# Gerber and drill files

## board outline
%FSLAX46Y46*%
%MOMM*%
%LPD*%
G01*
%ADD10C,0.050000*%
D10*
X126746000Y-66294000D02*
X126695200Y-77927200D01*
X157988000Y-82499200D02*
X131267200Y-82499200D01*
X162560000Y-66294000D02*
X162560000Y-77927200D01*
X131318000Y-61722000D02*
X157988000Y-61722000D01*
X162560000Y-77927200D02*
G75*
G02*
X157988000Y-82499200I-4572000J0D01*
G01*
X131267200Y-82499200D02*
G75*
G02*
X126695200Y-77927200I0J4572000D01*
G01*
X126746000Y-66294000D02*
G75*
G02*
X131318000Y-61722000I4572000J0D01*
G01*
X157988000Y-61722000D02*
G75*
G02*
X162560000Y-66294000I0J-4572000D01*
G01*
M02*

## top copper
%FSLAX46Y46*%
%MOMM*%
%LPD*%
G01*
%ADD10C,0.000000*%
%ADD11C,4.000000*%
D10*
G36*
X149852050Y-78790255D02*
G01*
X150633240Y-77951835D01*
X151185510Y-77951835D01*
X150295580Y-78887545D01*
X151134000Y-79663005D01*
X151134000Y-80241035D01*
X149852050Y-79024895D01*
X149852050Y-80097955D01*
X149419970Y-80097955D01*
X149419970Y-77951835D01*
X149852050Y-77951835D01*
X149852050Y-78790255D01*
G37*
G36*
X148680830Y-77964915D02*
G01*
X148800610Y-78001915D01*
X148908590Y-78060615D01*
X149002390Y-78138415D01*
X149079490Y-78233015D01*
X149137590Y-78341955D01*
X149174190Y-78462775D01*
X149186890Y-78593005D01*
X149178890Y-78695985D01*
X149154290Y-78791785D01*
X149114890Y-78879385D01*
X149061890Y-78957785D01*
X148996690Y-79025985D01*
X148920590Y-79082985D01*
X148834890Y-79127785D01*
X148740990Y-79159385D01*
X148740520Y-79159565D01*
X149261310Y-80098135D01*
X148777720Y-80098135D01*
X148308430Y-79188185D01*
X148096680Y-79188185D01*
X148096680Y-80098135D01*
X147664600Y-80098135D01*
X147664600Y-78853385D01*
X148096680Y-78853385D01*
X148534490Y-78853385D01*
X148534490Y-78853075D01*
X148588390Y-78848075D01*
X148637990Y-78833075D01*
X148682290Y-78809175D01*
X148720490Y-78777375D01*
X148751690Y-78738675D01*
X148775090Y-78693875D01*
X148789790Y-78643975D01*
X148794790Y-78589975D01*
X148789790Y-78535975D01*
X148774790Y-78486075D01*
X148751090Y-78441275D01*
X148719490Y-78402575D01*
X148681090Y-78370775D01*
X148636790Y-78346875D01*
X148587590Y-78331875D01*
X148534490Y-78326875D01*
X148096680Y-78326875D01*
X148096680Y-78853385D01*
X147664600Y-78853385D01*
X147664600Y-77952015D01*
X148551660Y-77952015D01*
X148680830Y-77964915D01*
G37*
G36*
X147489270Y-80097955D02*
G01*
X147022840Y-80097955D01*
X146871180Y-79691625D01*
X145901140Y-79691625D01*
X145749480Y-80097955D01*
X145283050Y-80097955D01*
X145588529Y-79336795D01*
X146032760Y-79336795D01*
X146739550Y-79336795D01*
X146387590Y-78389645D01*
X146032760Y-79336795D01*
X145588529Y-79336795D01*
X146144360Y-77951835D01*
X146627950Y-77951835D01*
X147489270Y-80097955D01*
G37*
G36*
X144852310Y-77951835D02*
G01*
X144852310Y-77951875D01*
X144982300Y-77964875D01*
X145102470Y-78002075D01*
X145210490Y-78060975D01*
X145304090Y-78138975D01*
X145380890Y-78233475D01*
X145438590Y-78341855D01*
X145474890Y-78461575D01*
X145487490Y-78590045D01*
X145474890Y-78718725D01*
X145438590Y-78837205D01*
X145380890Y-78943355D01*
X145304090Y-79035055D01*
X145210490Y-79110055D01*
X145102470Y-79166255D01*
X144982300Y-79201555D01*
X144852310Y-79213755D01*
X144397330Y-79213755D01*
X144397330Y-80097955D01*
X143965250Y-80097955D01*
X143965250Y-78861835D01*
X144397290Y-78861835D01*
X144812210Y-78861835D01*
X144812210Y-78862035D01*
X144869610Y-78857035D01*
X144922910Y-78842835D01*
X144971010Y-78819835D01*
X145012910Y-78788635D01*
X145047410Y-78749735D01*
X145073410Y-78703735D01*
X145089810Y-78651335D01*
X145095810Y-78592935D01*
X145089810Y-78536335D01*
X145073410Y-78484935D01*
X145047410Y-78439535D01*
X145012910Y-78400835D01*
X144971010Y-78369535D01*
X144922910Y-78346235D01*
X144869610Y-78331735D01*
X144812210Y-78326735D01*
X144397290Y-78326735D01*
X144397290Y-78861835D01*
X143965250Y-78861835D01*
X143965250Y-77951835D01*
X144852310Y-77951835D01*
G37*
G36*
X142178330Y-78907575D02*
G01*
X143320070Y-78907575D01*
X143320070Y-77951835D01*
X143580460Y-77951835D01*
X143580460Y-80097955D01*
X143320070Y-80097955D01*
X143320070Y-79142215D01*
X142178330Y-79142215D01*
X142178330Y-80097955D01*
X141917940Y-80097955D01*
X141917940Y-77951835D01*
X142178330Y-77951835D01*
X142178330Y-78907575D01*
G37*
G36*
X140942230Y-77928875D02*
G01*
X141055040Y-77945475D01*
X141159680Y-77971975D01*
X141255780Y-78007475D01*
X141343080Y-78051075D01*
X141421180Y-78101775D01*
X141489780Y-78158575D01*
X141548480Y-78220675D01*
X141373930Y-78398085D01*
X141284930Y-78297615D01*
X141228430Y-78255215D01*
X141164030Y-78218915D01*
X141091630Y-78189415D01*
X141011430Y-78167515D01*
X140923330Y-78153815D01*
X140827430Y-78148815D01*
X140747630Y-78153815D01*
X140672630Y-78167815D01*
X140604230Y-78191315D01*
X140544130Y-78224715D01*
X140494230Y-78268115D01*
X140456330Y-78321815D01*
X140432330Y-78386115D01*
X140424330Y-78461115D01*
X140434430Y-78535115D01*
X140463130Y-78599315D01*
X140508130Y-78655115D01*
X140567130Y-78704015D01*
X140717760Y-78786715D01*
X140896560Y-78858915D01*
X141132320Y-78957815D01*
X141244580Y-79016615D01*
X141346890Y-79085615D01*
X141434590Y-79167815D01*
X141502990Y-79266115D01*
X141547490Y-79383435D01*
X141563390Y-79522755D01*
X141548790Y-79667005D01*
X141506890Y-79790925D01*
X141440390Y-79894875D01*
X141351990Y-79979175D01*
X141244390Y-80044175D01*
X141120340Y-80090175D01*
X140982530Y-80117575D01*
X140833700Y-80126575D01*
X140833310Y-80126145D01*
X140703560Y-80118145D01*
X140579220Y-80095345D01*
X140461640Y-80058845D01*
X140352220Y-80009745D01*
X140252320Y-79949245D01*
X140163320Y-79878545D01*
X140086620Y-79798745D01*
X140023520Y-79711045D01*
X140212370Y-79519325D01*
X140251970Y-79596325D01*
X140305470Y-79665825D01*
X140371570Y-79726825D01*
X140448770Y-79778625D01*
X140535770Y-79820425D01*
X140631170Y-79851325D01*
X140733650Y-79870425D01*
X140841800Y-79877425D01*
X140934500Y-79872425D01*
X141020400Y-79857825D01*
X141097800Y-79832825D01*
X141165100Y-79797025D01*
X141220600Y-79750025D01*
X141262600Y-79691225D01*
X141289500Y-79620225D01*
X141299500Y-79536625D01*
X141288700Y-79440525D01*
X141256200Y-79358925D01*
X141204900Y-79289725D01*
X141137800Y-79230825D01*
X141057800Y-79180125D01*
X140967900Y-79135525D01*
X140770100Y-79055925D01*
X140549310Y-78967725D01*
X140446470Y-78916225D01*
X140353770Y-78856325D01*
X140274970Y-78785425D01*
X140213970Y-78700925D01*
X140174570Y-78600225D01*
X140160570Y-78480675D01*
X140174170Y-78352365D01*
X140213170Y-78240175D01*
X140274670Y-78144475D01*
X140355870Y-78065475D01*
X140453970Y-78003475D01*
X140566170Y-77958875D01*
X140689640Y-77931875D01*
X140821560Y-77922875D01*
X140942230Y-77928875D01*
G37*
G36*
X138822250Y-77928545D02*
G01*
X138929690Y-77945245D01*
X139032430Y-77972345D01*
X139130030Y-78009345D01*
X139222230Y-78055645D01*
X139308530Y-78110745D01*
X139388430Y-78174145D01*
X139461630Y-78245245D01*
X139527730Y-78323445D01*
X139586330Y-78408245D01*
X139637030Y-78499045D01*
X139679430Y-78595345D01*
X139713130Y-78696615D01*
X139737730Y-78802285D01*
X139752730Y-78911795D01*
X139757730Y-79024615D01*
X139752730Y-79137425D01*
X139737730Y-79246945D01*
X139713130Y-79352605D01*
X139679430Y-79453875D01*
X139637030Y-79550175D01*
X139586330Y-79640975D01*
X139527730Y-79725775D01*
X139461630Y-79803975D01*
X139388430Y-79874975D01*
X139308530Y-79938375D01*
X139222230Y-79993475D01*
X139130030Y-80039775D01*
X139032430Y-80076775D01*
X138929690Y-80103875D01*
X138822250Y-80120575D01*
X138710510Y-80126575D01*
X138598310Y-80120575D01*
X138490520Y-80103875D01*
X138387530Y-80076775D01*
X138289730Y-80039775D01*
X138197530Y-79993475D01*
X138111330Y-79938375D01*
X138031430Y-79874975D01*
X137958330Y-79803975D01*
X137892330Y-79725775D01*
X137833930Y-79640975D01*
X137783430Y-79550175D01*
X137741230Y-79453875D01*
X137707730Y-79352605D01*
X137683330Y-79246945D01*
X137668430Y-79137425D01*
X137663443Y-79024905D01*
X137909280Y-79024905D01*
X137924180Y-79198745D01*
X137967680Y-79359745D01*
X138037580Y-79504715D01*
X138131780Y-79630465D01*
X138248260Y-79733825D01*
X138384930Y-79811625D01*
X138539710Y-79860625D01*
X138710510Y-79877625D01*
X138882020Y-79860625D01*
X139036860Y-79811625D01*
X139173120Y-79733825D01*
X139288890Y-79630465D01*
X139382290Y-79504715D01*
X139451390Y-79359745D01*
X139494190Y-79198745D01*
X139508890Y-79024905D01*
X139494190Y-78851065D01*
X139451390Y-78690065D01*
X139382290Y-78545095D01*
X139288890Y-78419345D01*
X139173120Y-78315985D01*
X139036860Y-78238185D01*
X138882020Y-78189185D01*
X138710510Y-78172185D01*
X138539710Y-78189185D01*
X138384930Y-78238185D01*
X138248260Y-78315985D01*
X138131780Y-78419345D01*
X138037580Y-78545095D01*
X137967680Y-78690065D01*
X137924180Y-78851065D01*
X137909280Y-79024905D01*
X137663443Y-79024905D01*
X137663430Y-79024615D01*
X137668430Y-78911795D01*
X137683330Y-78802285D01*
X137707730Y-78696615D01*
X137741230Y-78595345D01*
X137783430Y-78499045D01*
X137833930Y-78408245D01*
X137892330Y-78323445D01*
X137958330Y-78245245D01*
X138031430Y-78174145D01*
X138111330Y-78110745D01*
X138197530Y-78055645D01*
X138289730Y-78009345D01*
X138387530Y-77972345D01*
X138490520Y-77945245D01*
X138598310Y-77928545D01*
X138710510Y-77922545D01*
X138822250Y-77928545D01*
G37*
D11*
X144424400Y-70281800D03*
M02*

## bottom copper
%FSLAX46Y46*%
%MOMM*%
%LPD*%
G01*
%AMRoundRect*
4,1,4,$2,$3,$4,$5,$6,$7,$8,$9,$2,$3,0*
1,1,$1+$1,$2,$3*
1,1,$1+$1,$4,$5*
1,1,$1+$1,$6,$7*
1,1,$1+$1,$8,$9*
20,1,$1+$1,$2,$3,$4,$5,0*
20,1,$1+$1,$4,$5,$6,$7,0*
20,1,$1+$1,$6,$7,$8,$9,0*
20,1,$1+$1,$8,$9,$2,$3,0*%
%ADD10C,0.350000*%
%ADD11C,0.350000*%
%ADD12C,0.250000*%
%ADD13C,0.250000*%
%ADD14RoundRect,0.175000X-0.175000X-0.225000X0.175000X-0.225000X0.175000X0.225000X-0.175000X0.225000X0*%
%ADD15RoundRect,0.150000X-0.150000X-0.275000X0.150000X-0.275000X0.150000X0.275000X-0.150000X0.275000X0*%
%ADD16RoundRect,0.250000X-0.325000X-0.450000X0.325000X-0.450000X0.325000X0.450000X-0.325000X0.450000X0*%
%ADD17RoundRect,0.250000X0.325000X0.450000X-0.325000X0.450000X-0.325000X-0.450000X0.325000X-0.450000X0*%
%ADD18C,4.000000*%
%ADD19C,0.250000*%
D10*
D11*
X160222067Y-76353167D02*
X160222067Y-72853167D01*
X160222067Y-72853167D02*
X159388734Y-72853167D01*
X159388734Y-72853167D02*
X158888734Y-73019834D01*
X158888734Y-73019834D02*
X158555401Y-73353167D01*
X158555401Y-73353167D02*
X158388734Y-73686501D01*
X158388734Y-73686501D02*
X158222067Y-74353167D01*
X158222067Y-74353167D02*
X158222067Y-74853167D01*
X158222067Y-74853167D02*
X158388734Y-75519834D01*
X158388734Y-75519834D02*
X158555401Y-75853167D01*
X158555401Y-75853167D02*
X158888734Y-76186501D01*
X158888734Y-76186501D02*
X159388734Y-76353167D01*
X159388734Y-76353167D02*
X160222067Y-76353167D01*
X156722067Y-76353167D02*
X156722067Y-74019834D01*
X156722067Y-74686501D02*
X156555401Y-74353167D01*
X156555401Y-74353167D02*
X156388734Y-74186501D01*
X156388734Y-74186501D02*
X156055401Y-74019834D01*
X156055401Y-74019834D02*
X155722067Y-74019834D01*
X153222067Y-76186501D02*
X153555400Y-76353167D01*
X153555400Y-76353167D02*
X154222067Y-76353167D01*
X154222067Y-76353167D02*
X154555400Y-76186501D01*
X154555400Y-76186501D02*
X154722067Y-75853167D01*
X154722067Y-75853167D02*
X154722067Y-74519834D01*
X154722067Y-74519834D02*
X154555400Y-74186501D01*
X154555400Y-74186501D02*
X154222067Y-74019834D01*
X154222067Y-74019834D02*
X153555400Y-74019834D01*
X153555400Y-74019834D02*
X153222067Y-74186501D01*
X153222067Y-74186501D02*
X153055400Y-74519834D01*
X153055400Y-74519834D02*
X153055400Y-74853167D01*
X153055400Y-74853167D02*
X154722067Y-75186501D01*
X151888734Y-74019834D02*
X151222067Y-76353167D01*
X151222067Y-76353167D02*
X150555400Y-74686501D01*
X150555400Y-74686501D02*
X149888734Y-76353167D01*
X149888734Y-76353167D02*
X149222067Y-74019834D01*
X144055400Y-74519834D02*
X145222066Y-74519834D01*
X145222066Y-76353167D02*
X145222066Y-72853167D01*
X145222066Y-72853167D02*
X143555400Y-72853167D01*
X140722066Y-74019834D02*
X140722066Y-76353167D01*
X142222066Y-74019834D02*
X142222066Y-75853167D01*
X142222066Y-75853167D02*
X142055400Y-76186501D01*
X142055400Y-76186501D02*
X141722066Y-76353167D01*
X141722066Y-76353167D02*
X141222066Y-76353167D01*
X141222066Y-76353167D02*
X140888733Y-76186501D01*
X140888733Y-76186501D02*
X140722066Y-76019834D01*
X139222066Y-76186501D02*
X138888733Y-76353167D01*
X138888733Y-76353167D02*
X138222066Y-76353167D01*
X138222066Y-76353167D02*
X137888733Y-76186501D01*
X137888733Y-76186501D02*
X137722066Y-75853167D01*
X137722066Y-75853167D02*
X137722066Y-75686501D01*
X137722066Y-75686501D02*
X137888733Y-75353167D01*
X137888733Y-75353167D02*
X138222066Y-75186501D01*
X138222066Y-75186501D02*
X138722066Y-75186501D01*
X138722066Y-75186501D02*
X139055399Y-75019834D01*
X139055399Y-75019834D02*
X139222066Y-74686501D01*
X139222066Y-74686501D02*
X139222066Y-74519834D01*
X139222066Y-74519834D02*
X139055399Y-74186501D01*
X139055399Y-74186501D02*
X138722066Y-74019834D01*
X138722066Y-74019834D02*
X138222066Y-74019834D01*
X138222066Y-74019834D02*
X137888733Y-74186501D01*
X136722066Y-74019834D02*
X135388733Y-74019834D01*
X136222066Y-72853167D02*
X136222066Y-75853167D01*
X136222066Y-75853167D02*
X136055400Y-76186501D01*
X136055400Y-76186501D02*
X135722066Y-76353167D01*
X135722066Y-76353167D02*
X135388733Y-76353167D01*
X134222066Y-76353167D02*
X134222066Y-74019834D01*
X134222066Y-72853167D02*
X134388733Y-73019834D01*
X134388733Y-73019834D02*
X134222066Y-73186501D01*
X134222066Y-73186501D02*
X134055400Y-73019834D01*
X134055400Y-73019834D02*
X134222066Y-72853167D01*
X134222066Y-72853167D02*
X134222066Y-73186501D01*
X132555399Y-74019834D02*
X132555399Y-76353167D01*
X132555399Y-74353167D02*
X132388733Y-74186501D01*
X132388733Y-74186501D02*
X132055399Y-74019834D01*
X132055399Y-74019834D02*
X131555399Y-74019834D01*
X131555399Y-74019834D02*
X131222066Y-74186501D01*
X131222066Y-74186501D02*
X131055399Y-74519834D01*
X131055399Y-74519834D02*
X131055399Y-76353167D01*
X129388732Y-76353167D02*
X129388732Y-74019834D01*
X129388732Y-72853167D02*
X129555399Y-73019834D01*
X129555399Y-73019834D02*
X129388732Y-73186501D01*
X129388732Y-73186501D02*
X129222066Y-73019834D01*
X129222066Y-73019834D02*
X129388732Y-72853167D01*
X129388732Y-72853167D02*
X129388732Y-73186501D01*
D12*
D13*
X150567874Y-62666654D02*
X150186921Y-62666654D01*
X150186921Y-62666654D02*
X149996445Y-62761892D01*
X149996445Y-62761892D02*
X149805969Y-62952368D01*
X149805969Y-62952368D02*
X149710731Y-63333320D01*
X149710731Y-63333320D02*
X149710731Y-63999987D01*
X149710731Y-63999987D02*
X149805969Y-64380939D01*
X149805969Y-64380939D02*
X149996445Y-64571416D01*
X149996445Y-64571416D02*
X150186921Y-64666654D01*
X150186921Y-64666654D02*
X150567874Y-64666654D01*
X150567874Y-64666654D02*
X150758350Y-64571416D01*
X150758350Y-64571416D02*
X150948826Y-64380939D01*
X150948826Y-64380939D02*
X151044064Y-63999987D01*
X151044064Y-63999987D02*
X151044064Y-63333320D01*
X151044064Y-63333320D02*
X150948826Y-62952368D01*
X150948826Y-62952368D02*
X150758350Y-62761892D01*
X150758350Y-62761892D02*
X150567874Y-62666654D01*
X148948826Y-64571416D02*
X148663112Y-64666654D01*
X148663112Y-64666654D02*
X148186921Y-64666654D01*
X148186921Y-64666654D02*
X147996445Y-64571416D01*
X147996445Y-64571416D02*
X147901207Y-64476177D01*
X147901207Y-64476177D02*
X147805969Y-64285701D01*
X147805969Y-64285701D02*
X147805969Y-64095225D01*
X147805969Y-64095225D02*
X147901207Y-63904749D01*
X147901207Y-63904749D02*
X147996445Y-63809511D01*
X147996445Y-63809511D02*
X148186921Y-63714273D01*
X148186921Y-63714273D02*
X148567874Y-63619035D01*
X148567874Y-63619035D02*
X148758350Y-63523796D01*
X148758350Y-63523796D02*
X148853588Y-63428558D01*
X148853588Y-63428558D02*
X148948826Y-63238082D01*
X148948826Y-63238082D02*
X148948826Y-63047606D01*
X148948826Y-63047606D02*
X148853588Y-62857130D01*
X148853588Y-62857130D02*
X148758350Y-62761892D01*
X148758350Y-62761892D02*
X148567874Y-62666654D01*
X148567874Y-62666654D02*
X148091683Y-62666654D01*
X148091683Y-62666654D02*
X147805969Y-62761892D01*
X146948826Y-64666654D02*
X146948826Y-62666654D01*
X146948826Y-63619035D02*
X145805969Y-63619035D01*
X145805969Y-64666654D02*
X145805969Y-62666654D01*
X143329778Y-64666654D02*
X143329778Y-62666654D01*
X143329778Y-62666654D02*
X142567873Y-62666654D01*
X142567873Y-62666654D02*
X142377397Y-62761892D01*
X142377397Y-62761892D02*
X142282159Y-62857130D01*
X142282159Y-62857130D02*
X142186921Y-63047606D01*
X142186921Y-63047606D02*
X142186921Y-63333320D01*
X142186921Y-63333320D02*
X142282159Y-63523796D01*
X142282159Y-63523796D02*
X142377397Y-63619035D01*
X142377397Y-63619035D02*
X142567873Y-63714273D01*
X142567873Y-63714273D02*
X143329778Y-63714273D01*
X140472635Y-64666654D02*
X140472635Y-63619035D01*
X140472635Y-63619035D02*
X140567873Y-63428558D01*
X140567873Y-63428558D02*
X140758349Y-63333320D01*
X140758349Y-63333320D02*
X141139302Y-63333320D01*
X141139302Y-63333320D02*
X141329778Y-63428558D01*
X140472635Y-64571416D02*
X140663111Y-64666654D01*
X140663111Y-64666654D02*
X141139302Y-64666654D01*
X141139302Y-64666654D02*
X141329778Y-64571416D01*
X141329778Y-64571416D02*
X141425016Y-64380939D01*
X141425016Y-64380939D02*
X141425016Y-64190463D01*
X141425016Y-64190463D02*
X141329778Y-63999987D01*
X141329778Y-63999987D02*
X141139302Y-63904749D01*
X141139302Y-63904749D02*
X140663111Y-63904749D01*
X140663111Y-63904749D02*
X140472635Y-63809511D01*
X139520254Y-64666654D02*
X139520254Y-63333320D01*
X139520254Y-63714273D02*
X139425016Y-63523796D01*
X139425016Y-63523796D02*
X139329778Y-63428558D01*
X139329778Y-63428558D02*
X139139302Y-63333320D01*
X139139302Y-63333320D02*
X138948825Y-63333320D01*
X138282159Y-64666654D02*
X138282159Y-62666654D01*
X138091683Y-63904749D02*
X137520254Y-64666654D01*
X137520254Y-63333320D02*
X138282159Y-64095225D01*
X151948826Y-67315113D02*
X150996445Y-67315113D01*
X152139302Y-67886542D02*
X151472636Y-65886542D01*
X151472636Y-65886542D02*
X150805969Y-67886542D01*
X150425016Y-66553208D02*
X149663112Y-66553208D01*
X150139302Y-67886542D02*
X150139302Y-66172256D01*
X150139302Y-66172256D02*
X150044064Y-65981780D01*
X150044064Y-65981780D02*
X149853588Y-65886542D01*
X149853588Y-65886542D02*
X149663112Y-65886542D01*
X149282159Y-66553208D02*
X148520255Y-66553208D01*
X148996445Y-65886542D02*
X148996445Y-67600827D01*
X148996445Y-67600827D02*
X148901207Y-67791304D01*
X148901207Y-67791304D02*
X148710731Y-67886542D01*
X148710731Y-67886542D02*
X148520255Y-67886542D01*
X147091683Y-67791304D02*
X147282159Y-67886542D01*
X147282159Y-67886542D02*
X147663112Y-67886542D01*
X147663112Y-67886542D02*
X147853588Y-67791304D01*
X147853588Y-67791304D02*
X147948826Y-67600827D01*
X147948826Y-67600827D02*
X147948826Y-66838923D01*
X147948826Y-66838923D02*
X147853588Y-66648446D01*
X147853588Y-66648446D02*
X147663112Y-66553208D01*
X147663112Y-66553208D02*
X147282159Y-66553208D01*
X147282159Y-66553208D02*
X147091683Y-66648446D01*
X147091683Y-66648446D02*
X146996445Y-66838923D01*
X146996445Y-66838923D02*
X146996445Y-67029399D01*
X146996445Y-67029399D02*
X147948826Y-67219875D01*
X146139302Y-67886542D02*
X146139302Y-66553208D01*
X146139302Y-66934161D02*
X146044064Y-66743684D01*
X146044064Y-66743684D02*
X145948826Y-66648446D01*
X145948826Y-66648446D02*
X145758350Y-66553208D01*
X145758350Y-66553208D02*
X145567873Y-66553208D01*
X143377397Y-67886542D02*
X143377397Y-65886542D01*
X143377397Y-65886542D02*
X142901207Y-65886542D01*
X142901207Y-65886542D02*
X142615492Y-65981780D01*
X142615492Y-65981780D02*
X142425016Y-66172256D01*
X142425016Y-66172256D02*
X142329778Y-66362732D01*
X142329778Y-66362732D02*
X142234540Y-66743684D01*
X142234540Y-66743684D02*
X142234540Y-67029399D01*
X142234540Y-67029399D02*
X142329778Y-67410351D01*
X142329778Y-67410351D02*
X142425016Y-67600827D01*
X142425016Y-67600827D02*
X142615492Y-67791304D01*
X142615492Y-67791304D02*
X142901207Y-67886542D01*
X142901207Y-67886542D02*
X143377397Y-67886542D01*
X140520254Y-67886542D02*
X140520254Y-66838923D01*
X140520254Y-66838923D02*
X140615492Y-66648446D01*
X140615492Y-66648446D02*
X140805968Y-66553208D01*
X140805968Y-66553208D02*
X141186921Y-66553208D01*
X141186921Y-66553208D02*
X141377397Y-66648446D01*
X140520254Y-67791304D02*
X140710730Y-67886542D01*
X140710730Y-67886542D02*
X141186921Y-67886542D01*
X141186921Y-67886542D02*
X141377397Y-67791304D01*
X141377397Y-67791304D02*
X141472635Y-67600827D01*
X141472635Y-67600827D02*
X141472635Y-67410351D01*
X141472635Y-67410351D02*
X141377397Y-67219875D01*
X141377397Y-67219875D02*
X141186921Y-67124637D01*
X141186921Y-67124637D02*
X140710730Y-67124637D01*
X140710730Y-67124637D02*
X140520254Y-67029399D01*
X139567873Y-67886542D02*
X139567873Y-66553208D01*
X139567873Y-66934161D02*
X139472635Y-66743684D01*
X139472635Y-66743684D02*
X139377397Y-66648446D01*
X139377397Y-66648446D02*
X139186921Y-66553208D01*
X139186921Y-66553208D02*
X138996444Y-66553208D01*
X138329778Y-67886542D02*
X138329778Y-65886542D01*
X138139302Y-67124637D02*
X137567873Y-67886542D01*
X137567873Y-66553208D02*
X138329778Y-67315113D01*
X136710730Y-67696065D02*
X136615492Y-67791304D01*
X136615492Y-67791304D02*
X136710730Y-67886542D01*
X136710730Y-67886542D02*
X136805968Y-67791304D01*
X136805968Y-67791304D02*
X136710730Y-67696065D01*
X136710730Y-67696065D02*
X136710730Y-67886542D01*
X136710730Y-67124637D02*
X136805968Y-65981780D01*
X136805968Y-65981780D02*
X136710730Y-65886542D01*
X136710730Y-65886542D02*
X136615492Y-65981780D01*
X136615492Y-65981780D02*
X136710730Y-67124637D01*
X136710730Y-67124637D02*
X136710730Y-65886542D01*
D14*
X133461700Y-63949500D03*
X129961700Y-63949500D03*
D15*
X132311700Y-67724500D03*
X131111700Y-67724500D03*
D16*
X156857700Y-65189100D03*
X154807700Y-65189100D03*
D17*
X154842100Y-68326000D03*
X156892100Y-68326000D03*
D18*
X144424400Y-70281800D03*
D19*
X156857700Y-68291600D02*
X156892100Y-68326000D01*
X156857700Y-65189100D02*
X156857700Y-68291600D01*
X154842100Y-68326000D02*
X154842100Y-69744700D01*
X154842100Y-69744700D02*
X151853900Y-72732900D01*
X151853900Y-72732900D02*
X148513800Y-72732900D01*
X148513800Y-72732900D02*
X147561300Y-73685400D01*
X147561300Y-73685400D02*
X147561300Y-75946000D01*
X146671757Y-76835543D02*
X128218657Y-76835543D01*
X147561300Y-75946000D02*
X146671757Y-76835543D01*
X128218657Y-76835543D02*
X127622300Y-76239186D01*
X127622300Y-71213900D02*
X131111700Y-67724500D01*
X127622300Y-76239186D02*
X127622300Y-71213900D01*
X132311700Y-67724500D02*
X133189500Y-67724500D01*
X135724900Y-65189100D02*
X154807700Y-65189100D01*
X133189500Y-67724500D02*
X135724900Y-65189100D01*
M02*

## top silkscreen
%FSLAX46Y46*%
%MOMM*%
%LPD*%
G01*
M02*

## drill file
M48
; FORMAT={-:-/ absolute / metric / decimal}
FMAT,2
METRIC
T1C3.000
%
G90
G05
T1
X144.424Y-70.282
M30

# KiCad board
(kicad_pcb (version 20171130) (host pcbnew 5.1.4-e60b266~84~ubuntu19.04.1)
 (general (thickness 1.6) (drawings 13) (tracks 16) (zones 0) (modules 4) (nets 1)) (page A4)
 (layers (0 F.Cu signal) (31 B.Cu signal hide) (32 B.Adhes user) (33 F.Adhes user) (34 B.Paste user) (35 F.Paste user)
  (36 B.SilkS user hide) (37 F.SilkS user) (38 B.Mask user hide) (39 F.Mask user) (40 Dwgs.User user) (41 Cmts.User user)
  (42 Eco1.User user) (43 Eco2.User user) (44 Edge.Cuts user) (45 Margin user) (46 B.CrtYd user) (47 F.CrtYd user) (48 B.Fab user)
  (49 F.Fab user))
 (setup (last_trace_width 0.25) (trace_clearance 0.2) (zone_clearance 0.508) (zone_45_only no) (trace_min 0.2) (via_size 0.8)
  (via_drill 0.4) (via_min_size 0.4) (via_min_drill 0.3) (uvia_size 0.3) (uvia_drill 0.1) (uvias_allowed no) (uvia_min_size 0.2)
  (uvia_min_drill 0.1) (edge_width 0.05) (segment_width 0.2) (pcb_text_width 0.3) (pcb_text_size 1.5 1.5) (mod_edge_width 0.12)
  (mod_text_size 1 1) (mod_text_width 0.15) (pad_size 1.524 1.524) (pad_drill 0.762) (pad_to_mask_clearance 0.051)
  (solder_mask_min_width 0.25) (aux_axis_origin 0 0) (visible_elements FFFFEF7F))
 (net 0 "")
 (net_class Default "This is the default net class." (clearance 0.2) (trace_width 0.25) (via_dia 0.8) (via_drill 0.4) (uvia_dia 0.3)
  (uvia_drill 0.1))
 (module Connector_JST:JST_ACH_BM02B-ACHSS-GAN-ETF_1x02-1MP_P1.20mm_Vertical (layer B.Cu) (at 131.7117 65.8495)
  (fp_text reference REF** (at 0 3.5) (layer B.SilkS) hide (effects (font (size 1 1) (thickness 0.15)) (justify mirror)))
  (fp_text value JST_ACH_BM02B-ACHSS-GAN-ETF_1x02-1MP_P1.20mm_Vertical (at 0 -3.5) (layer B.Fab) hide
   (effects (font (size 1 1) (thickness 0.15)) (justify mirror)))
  (pad MP smd roundrect (at 1.75 -1.9) (size 0.7 0.8) (layers B.Cu B.Paste B.Mask) (roundrect_rratio 0.25))
  (pad MP smd roundrect (at -1.75 -1.9) (size 0.7 0.8) (layers B.Cu B.Paste B.Mask) (roundrect_rratio 0.25))
  (pad 2 smd roundrect (at 0.6 1.875) (size 0.6 0.85) (layers B.Cu B.Paste B.Mask) (roundrect_rratio 0.25))
  (pad 1 smd roundrect (at -0.6 1.875) (size 0.6 0.85) (layers B.Cu B.Paste B.Mask) (roundrect_rratio 0.25)))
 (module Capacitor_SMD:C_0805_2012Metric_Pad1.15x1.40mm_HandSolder (layer B.Cu) (at 155.8327 65.1891)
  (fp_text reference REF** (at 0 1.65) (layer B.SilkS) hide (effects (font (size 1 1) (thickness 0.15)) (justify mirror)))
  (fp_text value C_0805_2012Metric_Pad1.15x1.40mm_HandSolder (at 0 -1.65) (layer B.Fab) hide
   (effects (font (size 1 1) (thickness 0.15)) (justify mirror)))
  (pad 2 smd roundrect (at 1.025 0) (size 1.15 1.4) (layers B.Cu B.Paste B.Mask) (roundrect_rratio 0.217391))
  (pad 1 smd roundrect (at -1.025 0) (size 1.15 1.4) (layers B.Cu B.Paste B.Mask) (roundrect_rratio 0.217391)))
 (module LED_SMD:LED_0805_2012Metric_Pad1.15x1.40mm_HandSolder (layer B.Cu) (at 155.8671 68.326 180)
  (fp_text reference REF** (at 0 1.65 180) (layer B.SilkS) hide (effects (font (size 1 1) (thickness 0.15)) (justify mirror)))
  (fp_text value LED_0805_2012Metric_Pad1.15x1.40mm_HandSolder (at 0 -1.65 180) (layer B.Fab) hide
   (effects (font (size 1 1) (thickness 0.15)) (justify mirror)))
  (pad 2 smd roundrect (at 1.025 0 180) (size 1.15 1.4) (layers B.Cu B.Paste B.Mask) (roundrect_rratio 0.217391))
  (pad 1 smd roundrect (at -1.025 0 180) (size 1.15 1.4) (layers B.Cu B.Paste B.Mask) (roundrect_rratio 0.217391)))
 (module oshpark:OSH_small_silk (layer F.Cu) (at 144.4244 71.8312)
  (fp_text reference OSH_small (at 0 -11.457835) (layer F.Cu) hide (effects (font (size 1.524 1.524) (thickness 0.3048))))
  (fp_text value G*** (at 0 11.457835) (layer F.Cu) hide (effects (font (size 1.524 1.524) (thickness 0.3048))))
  (fp_poly
   (pts (xy 6.76111 6.120635) (xy 6.20884 6.120635) (xy 5.42765 6.959055) (xy 5.42765 6.120635) (xy 4.99557 6.120635) (xy 4.99557 8.266755)
    (xy 5.42765 8.266755) (xy 5.42765 7.193695) (xy 6.7096 8.409835) (xy 6.7096 7.831805) (xy 5.87118 7.056345) (xy 6.76111 6.120635))
   (layer F.Cu) (width 0))
  (fp_poly
   (pts (xy 4.31659 7.328185) (xy 4.11009 7.022185) (xy 3.67228 7.022185) (xy 3.67228 6.495675) (xy 4.11009 6.495675) (xy 4.16319 6.500675)
    (xy 4.21239 6.515675) (xy 4.25669 6.539575) (xy 4.29509 6.571375) (xy 4.32669 6.610075) (xy 4.35039 6.654875) (xy 4.36539 6.704775)
    (xy 4.37039 6.758775) (xy 4.36539 6.812775) (xy 4.35069 6.862675) (xy 4.32729 6.907475) (xy 4.29609 6.946175) (xy 4.25789 6.977975)
    (xy 4.21359 7.001875) (xy 4.16399 7.016875) (xy 4.11009 7.021875) (xy 4.11009 7.022185) (xy 4.31659 7.328185) (xy 4.41049 7.296585)
    (xy 4.49619 7.251785) (xy 4.57229 7.194785) (xy 4.63749 7.126585) (xy 4.69049 7.048185) (xy 4.72989 6.960585) (xy 4.75449 6.864785)
    (xy 4.76249 6.761805) (xy 4.74979 6.631575) (xy 4.71319 6.510755) (xy 4.65509 6.401815) (xy 4.57799 6.307215) (xy 4.48419 6.229415)
    (xy 4.37621 6.170715) (xy 4.25643 6.133715) (xy 4.12726 6.120815) (xy 3.2402 6.120815) (xy 3.2402 8.266935) (xy 3.67228 8.266935)
    (xy 3.67228 7.356985) (xy 3.88403 7.356985) (xy 4.35332 8.266935) (xy 4.83691 8.266935) (xy 4.31612 7.328365) (xy 4.31659 7.328185))
   (layer F.Cu) (width 0))
  (fp_poly
   (pts (xy 2.59844 8.266755) (xy 1.96319 6.558445) (xy 2.31515 7.505595) (xy 1.60836 7.505595) (xy 1.96319 6.558445) (xy 2.59844 8.266755)
    (xy 3.06487 8.266755) (xy 2.20355 6.120635) (xy 1.71996 6.120635) (xy 0.85865 8.266755) (xy 1.32508 8.266755) (xy 1.47674 7.860425)
    (xy 2.44678 7.860425) (xy 2.59844 8.266755))
   (layer F.Cu) (width 0))
  (fp_poly
   (pts (xy 0.42791 6.120635) (xy -0.02711 6.495535) (xy 0.38781 6.495535) (xy 0.44521 6.500535) (xy 0.49851 6.515035) (xy 0.54661 6.538335)
    (xy 0.58851 6.569635) (xy 0.62301 6.608335) (xy 0.64901 6.653735) (xy 0.66541 6.705135) (xy 0.67141 6.761735) (xy 0.66541 6.820135)
    (xy 0.64901 6.872535) (xy 0.62301 6.918535) (xy 0.58851 6.957435) (xy 0.54661 6.988635) (xy 0.49851 7.011635) (xy 0.44521 7.025835)
    (xy 0.38781 7.030835) (xy 0.38781 7.030635) (xy -0.02711 7.030635) (xy -0.02711 6.495535) (xy 0.42791 6.120635) (xy -0.45915 6.120635)
    (xy -0.45915 8.266755) (xy -0.02707 8.266755) (xy -0.02707 7.382555) (xy 0.42791 7.382555) (xy 0.5579 7.370355) (xy 0.67807 7.335055)
    (xy 0.78609 7.278855) (xy 0.87969 7.203855) (xy 0.95649 7.112155) (xy 1.01419 7.006005) (xy 1.05049 6.887525) (xy 1.06309 6.758845)
    (xy 1.05049 6.630375) (xy 1.01419 6.510655) (xy 0.95649 6.402275) (xy 0.87969 6.307775) (xy 0.78609 6.229775) (xy 0.67807 6.170875)
    (xy 0.5579 6.133675) (xy 0.42791 6.120675) (xy 0.42791 6.120635))
   (layer F.Cu) (width 0))
  (fp_poly
   (pts (xy -1.10433 6.120635) (xy -1.10433 7.076375) (xy -2.24607 7.076375) (xy -2.24607 6.120635) (xy -2.50646 6.120635)
    (xy -2.50646 8.266755) (xy -2.24607 8.266755) (xy -2.24607 7.311015) (xy -1.10433 7.311015) (xy -1.10433 8.266755)
    (xy -0.84394 8.266755) (xy -0.84394 6.120635) (xy -1.10433 6.120635))
   (layer F.Cu) (width 0))
  (fp_poly
   (pts (xy -3.5907 8.295375) (xy -3.44187 8.286375) (xy -3.30406 8.258975) (xy -3.18001 8.212975) (xy -3.07241 8.147975)
    (xy -2.98401 8.063675) (xy -2.91751 7.959725) (xy -2.87561 7.835805) (xy -2.86101 7.691555) (xy -2.87691 7.552235)
    (xy -2.92141 7.434915) (xy -2.98981 7.336615) (xy -3.07751 7.254415) (xy -3.17982 7.185415) (xy -3.29208 7.126615)
    (xy -3.52784 7.027715) (xy -3.70664 6.955515) (xy -3.85727 6.872815) (xy -3.91627 6.823915) (xy -3.96127 6.768115)
    (xy -3.98997 6.703915) (xy -4.00007 6.629915) (xy -3.99207 6.554915) (xy -3.96807 6.490615) (xy -3.93017 6.436915)
    (xy -3.88027 6.393515) (xy -3.82017 6.360115) (xy -3.75177 6.336615) (xy -3.67677 6.322615) (xy -3.59697 6.317615)
    (xy -3.50107 6.322615) (xy -3.41297 6.336315) (xy -3.33277 6.358215) (xy -3.26037 6.387715) (xy -3.19597 6.424015)
    (xy -3.13947 6.466415) (xy -3.05047 6.566885) (xy -2.87592 6.389475) (xy -2.93462 6.327375) (xy -3.00322 6.270575)
    (xy -3.08132 6.219875) (xy -3.16862 6.176275) (xy -3.26472 6.140775) (xy -3.36936 6.114275) (xy -3.48217 6.097675)
    (xy -3.60284 6.091675) (xy -3.73476 6.100675) (xy -3.85823 6.127675) (xy -3.97043 6.172275) (xy -4.06853 6.234275)
    (xy -4.14973 6.313275) (xy -4.21123 6.408975) (xy -4.25023 6.521165) (xy -4.26383 6.649475) (xy -4.24983 6.769025)
    (xy -4.21043 6.869725) (xy -4.14943 6.954225) (xy -4.07063 7.025125) (xy -3.97793 7.085025) (xy -3.87509 7.136525) (xy -3.6543 7.224725)
    (xy -3.4565 7.304325) (xy -3.3666 7.348925) (xy -3.2866 7.399625) (xy -3.2195 7.458525) (xy -3.1682 7.527725) (xy -3.1357 7.609325)
    (xy -3.1249 7.705425) (xy -3.1349 7.789025) (xy -3.1618 7.860025) (xy -3.2038 7.918825) (xy -3.2593 7.965825) (xy -3.3266 8.001625)
    (xy -3.404 8.026625) (xy -3.4899 8.041225) (xy -3.5826 8.046225) (xy -3.69075 8.039225) (xy -3.79323 8.020125) (xy -3.88863 7.989225)
    (xy -3.97563 7.947425) (xy -4.05283 7.895625) (xy -4.11893 7.834625) (xy -4.17243 7.765125) (xy -4.21203 7.688125)
    (xy -4.40088 7.879845) (xy -4.33778 7.967545) (xy -4.26108 8.047345) (xy -4.17208 8.118045) (xy -4.07218 8.178545)
    (xy -3.96276 8.227645) (xy -3.84518 8.264145) (xy -3.72084 8.286945) (xy -3.59109 8.294945) (xy -3.5907 8.295375))
   (layer F.Cu) (width 0))
  (fp_poly
   (pts (xy -5.71389 8.295375) (xy -5.71389 8.046425) (xy -5.88469 8.029425) (xy -6.03947 7.980425) (xy -6.17614 7.902625)
    (xy -6.29262 7.799265) (xy -6.38682 7.673515) (xy -6.45672 7.528545) (xy -6.50022 7.367545) (xy -6.51512 7.193705)
    (xy -6.50022 7.019865) (xy -6.45672 6.858865) (xy -6.38682 6.713895) (xy -6.29262 6.588145) (xy -6.17614 6.484785)
    (xy -6.03947 6.406985) (xy -5.88469 6.357985) (xy -5.71389 6.340985) (xy -5.54238 6.357985) (xy -5.38754 6.406985)
    (xy -5.25128 6.484785) (xy -5.13551 6.588145) (xy -5.04211 6.713895) (xy -4.97301 6.858865) (xy -4.93021 7.019865)
    (xy -4.91551 7.193705) (xy -4.93021 7.367545) (xy -4.97301 7.528545) (xy -5.04211 7.673515) (xy -5.13551 7.799265)
    (xy -5.25128 7.902625) (xy -5.38754 7.980425) (xy -5.54238 8.029425) (xy -5.71389 8.046425) (xy -5.71389 8.295375)
    (xy -5.60215 8.289375) (xy -5.49471 8.272675) (xy -5.39197 8.245575) (xy -5.29437 8.208575) (xy -5.20217 8.162275)
    (xy -5.11587 8.107175) (xy -5.03597 8.043775) (xy -4.96277 7.972775) (xy -4.89667 7.894575) (xy -4.83807 7.809775)
    (xy -4.78737 7.718975) (xy -4.74497 7.622675) (xy -4.71127 7.521405) (xy -4.68667 7.415745) (xy -4.67167 7.306225)
    (xy -4.66667 7.193415) (xy -4.67167 7.080595) (xy -4.68667 6.971085) (xy -4.71127 6.865415) (xy -4.74497 6.764145)
    (xy -4.78737 6.667845) (xy -4.83807 6.577045) (xy -4.89667 6.492245) (xy -4.96277 6.414045) (xy -5.03597 6.342945)
    (xy -5.11587 6.279545) (xy -5.20217 6.224445) (xy -5.29437 6.178145) (xy -5.39197 6.141145) (xy -5.49471 6.114045)
    (xy -5.60215 6.097345) (xy -5.71389 6.091345) (xy -5.82609 6.097345) (xy -5.93388 6.114045) (xy -6.03687 6.141145)
    (xy -6.13467 6.178145) (xy -6.22687 6.224445) (xy -6.31307 6.279545) (xy -6.39297 6.342945) (xy -6.46607 6.414045)
    (xy -6.53207 6.492245) (xy -6.59047 6.577045) (xy -6.64097 6.667845) (xy -6.68317 6.764145) (xy -6.71667 6.865415)
    (xy -6.74107 6.971085) (xy -6.75597 7.080595) (xy -6.76097 7.193415) (xy -6.75597 7.306225) (xy -6.74107 7.415745)
    (xy -6.71667 7.521405) (xy -6.68317 7.622675) (xy -6.64097 7.718975) (xy -6.59047 7.809775) (xy -6.53207 7.894575)
    (xy -6.46607 7.972775) (xy -6.39297 8.043775) (xy -6.31307 8.107175) (xy -6.22687 8.162275) (xy -6.13467 8.208575)
    (xy -6.03687 8.245575) (xy -5.93388 8.272675) (xy -5.82609 8.289375) (xy -5.71389 8.295375))
   (layer F.Cu) (width 0)))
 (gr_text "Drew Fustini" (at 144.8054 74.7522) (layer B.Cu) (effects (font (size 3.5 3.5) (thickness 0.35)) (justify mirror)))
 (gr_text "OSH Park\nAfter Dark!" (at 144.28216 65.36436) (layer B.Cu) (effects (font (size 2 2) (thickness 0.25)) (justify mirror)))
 (gr_line (start 126.746 66.294) (end 126.6952 77.9272) (layer Edge.Cuts) (width 0.05))
 (gr_line (start 157.988 82.4992) (end 131.2672 82.4992) (layer Edge.Cuts) (width 0.05))
 (gr_line (start 162.56 66.294) (end 162.56 77.9272) (layer Edge.Cuts) (width 0.05))
 (gr_line (start 131.318 61.722) (end 157.988 61.722) (layer Edge.Cuts) (width 0.05))
 (gr_arc (start 157.988 77.9272) (end 157.988 82.4992) (angle -90) (layer Edge.Cuts) (width 0.05))
 (gr_arc (start 131.2672 77.9272) (end 126.6952 77.9272) (angle -90) (layer Edge.Cuts) (width 0.05))
 (gr_arc (start 131.318 66.294) (end 131.318 61.722) (angle -90) (layer Edge.Cuts) (width 0.05))
 (gr_arc (start 157.988 66.294) (end 162.56 66.294) (angle -90) (layer Edge.Cuts) (width 0.05))
 (segment (start 156.8577 68.2916) (end 156.8921 68.326) (width 0.25) (layer B.Cu) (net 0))
 (segment (start 156.8577 65.1891) (end 156.8577 68.2916) (width 0.25) (layer B.Cu) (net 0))
 (segment (start 154.8421 68.326) (end 154.8421 69.7447) (width 0.25) (layer B.Cu) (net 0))
 (segment (start 154.8421 69.7447) (end 151.8539 72.7329) (width 0.25) (layer B.Cu) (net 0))
 (segment (start 151.8539 72.7329) (end 148.5138 72.7329) (width 0.25) (layer B.Cu) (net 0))
 (segment (start 148.5138 72.7329) (end 147.5613 73.6854) (width 0.25) (layer B.Cu) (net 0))
 (segment (start 147.5613 73.6854) (end 147.5613 75.946) (width 0.25) (layer B.Cu) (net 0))
 (segment (start 146.671757 76.835543) (end 128.218657 76.835543) (width 0.25) (layer B.Cu) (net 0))
 (segment (start 147.5613 75.946) (end 146.671757 76.835543) (width 0.25) (layer B.Cu) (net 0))
 (segment (start 128.218657 76.835543) (end 127.6223 76.239186) (width 0.25) (layer B.Cu) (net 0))
 (segment (start 127.6223 71.2139) (end 131.1117 67.7245) (width 0.25) (layer B.Cu) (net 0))
 (segment (start 127.6223 76.239186) (end 127.6223 71.2139) (width 0.25) (layer B.Cu) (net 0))
 (segment (start 132.3117 67.7245) (end 133.1895 67.7245) (width 0.25) (layer B.Cu) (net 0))
 (segment (start 135.7249 65.1891) (end 154.8077 65.1891) (width 0.25) (layer B.Cu) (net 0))
 (segment (start 133.1895 67.7245) (end 135.7249 65.1891) (width 0.25) (layer B.Cu) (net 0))
 (via (at 144.4244 70.2818) (size 4) (drill 3) (layers F.Cu B.Cu) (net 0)))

